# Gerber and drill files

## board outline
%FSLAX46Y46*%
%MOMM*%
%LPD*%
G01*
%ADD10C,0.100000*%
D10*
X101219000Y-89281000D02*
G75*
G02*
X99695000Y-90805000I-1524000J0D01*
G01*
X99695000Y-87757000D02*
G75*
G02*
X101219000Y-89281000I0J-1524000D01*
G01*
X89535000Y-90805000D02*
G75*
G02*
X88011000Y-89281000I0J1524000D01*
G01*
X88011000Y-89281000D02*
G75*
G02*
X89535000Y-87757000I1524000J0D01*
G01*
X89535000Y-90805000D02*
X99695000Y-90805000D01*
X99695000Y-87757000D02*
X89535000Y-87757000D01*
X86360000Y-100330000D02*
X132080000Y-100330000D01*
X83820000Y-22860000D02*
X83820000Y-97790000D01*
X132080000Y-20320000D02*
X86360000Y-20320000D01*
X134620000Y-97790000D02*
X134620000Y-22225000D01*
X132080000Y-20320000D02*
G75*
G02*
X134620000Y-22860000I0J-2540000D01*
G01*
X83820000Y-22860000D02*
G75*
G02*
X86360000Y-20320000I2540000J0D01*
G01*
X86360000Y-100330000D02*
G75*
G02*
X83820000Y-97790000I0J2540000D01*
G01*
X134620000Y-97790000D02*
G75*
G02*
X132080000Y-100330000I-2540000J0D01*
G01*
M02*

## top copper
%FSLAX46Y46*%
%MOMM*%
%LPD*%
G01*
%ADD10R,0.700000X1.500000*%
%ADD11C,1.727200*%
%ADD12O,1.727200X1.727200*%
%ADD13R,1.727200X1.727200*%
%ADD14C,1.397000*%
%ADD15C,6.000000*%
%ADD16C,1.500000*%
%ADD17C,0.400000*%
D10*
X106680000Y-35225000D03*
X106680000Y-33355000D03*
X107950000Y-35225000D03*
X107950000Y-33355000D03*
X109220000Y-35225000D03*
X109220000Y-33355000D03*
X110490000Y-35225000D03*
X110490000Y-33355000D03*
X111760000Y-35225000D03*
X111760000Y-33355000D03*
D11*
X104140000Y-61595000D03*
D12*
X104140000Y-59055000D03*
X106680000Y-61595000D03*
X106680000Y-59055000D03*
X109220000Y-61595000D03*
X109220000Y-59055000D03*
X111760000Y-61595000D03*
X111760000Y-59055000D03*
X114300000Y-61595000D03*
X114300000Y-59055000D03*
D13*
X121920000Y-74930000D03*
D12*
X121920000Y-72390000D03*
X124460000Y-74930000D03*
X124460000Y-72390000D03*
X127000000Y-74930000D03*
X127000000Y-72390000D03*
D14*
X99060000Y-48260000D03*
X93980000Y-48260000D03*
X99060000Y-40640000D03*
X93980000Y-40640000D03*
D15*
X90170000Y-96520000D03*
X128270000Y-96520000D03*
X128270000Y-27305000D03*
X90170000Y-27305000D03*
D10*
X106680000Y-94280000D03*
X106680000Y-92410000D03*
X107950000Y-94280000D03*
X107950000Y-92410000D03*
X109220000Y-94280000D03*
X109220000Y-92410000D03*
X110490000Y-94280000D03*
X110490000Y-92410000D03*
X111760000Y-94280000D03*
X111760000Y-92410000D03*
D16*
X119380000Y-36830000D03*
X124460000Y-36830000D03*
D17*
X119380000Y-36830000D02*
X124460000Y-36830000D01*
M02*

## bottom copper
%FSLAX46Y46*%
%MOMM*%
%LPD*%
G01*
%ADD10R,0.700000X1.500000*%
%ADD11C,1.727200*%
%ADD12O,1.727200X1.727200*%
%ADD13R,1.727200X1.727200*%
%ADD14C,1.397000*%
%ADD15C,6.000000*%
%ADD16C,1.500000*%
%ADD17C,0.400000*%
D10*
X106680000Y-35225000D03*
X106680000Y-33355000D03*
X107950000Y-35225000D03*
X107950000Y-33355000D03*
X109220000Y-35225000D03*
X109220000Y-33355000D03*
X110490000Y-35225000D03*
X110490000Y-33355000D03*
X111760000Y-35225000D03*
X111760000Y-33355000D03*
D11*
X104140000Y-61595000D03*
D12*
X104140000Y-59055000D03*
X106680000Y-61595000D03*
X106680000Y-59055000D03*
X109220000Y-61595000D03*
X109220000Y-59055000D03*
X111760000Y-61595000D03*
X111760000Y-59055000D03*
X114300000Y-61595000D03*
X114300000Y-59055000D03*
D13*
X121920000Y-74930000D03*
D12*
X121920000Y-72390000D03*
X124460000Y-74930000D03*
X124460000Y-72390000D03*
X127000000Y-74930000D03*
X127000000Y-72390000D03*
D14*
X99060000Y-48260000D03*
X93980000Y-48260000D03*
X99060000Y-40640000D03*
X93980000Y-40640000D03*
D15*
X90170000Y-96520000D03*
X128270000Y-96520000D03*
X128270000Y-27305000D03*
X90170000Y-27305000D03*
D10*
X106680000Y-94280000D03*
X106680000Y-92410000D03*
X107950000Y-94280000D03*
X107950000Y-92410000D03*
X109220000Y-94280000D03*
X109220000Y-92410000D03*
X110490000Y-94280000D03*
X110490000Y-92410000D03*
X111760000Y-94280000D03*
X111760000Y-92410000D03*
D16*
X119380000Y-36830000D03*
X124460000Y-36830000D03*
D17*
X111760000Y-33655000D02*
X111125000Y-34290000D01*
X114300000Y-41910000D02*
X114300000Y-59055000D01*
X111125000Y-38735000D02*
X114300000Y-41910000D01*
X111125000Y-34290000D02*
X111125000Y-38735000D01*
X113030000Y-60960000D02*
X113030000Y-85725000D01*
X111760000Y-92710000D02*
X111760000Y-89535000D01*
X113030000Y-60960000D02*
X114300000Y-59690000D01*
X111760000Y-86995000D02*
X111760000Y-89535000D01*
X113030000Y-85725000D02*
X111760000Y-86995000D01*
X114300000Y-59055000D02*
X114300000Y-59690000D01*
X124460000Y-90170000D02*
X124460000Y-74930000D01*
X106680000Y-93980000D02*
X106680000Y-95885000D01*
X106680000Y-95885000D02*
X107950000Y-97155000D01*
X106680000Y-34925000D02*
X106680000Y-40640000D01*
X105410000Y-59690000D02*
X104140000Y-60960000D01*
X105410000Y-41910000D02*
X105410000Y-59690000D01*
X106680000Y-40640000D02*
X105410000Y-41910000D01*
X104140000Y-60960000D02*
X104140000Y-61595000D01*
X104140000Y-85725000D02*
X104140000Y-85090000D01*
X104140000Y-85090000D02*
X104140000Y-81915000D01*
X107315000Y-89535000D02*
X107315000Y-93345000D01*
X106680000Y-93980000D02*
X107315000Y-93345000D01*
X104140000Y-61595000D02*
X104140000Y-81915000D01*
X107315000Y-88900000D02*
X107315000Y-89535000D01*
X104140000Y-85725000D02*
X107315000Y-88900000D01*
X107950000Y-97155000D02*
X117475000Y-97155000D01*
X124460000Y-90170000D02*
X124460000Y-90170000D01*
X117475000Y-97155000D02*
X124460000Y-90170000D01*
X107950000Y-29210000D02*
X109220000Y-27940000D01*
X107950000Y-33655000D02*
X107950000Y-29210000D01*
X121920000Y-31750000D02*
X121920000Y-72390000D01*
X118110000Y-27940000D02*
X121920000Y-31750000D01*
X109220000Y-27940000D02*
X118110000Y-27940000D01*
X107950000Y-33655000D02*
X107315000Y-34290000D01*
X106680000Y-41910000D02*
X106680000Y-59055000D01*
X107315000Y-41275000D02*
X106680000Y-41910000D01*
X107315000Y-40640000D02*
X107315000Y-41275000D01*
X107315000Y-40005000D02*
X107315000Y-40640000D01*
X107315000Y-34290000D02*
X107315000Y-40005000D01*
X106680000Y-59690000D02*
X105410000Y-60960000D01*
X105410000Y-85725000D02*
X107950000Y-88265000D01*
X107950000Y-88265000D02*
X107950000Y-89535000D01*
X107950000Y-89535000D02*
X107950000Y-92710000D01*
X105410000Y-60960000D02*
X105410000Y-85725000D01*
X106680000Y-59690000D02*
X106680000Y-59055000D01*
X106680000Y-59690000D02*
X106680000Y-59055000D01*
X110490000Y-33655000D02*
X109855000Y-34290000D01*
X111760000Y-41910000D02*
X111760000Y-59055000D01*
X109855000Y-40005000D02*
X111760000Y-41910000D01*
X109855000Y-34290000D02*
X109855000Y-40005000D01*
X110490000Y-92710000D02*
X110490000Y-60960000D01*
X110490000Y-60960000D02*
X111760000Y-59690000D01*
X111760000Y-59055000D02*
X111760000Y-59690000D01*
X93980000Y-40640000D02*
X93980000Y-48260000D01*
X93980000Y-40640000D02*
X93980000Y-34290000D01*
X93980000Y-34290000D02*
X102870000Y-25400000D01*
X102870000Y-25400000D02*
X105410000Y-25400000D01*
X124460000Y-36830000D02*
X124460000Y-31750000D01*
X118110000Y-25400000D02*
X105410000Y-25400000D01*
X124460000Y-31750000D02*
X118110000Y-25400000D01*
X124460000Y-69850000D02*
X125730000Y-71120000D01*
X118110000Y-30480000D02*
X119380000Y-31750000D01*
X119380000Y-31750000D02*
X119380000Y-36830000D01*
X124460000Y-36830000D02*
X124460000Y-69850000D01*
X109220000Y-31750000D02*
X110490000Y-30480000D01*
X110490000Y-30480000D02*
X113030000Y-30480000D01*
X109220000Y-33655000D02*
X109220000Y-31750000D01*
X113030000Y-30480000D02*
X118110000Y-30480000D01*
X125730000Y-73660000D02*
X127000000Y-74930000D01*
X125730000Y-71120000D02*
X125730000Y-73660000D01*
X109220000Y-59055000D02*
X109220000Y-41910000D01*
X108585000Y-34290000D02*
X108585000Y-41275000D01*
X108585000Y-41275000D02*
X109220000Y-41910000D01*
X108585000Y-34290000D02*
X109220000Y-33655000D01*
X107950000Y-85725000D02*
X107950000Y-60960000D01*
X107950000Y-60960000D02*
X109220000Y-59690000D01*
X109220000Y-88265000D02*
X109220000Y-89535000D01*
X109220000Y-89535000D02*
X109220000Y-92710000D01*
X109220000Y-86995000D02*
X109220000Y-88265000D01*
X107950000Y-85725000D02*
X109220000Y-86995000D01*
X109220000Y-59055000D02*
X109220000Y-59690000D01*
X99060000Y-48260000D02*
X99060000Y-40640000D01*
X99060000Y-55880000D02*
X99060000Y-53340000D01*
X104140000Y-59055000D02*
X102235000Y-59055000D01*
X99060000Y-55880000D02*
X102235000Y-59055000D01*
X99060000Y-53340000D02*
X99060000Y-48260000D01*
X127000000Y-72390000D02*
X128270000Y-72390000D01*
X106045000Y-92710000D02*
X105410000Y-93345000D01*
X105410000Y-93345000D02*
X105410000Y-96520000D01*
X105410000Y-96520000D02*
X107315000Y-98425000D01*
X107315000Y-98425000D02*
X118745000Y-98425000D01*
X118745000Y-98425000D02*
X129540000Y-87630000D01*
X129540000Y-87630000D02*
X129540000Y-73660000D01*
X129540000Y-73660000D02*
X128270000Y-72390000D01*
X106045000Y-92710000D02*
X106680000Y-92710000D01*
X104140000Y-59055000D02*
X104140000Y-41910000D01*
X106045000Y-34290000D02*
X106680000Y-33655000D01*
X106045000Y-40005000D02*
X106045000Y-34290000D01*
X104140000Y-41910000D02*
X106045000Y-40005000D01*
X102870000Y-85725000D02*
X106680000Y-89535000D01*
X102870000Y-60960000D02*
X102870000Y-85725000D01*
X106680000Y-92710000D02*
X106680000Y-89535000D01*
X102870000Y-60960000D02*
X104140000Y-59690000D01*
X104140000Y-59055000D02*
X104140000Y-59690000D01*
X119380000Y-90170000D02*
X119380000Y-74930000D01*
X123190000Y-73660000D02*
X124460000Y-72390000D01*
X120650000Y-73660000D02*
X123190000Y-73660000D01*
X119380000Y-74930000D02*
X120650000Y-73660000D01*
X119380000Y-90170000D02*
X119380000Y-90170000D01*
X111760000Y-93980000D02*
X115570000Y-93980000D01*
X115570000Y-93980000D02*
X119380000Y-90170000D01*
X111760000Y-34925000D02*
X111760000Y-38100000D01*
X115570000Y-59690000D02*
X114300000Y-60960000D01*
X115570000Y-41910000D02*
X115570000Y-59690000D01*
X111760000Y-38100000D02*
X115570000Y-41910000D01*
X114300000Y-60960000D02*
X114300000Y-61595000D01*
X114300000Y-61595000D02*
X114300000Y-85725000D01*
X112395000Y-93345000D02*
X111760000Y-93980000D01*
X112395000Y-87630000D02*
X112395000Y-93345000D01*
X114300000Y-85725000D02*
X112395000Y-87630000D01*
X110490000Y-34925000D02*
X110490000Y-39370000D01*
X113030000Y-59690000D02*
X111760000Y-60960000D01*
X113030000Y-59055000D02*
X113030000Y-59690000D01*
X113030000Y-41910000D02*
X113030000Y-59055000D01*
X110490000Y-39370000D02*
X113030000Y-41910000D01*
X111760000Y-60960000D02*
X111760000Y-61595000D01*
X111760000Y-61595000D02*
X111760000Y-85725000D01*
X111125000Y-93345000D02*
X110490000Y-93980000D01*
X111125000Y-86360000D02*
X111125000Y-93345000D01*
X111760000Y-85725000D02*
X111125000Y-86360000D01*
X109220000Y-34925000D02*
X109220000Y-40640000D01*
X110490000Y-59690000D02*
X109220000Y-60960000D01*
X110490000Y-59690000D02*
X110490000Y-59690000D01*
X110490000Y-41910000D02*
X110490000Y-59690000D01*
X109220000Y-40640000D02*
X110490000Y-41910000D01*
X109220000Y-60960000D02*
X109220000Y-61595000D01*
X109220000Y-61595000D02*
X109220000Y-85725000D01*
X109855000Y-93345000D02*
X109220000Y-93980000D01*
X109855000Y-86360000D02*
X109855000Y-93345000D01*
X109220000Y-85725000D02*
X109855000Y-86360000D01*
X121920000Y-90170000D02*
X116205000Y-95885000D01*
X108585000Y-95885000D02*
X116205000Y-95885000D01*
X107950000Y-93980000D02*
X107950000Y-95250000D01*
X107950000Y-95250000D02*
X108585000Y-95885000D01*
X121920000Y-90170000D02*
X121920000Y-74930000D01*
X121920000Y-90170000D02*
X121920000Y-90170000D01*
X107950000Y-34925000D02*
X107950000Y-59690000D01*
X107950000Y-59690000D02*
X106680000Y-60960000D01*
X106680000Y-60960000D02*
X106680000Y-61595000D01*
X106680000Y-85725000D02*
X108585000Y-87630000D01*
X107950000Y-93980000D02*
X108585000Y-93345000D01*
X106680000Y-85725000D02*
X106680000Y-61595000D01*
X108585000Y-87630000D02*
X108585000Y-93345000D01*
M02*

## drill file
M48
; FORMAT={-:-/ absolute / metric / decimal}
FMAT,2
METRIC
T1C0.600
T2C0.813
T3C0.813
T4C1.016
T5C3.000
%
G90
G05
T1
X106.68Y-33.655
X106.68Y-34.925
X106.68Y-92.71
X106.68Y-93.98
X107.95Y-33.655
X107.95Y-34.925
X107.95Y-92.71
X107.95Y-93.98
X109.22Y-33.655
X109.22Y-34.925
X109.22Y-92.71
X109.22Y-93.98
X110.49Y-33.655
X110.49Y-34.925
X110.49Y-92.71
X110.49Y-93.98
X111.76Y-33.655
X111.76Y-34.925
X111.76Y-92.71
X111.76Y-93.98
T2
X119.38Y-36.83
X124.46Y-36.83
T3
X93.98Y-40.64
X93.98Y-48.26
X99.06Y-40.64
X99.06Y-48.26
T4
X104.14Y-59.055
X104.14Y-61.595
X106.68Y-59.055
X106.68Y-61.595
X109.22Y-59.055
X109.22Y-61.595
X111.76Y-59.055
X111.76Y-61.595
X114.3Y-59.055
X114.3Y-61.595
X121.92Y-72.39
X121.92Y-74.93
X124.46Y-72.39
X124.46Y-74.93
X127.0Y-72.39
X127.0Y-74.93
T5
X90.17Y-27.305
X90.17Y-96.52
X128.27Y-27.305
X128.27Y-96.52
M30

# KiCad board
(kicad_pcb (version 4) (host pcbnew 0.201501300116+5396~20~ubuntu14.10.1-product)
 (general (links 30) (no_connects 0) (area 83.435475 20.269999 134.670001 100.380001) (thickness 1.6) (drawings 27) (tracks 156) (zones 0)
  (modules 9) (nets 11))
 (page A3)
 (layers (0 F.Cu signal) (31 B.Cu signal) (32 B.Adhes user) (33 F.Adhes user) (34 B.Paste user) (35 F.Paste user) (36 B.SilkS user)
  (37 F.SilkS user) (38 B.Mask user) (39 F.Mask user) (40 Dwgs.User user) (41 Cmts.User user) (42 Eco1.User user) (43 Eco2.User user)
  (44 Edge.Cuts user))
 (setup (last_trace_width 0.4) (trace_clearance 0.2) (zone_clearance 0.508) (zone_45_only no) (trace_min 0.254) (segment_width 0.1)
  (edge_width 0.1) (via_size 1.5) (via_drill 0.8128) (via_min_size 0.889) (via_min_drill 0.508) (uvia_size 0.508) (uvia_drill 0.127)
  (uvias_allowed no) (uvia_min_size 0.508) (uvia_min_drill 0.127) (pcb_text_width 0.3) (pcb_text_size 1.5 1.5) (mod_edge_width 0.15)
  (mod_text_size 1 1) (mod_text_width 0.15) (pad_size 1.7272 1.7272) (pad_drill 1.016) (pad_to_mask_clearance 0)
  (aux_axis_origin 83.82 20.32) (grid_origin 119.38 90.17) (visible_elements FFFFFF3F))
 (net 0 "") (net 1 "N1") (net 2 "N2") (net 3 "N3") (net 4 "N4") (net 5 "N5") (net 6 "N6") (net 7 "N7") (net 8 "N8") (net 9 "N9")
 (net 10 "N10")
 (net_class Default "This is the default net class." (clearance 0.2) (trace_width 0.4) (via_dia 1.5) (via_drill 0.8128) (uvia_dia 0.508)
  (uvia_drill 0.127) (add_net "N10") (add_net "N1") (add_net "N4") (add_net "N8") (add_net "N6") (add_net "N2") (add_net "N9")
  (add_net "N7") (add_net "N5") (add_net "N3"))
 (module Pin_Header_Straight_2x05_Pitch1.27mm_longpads (layer F.Cu) (at 109.22 34.29)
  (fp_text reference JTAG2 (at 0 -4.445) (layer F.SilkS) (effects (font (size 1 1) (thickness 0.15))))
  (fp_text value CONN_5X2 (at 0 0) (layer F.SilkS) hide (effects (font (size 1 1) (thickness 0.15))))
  (pad 1 thru_hole rect (at -2.54 0.635) (size 0.7 1.5) (drill 0.6 (offset 0 0.3)) (layers *.Cu *.Mask F.SilkS) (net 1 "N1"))
  (pad 2 thru_hole rect (at -2.54 -0.635) (size 0.7 1.5) (drill 0.6 (offset 0 -0.3)) (layers *.Cu *.Mask F.SilkS) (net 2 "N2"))
  (pad 3 thru_hole rect (at -1.27 0.635) (size 0.7 1.5) (drill 0.6 (offset 0 0.3)) (layers *.Cu *.Mask F.SilkS) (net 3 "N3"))
  (pad 4 thru_hole rect (at -1.27 -0.635) (size 0.7 1.5) (drill 0.6 (offset 0 -0.3)) (layers *.Cu *.Mask F.SilkS) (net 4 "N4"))
  (pad 5 thru_hole rect (at 0 0.635) (size 0.7 1.5) (drill 0.6 (offset 0 0.3)) (layers *.Cu *.Mask F.SilkS) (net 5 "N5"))
  (pad 6 thru_hole rect (at 0 -0.635) (size 0.7 1.5) (drill 0.6 (offset 0 -0.3)) (layers *.Cu *.Mask F.SilkS) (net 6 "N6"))
  (pad 7 thru_hole rect (at 1.27 0.635) (size 0.7 1.5) (drill 0.6 (offset 0 0.3)) (layers *.Cu *.Mask F.SilkS) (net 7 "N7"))
  (pad 8 thru_hole rect (at 1.27 -0.635) (size 0.7 1.5) (drill 0.6 (offset 0 -0.3)) (layers *.Cu *.Mask F.SilkS) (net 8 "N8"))
  (pad 9 thru_hole rect (at 2.54 0.635) (size 0.7 1.5) (drill 0.6 (offset 0 0.3)) (layers *.Cu *.Mask F.SilkS) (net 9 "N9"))
  (pad 10 thru_hole rect (at 2.54 -0.635) (size 0.7 1.5) (drill 0.6 (offset 0 -0.3)) (layers *.Cu *.Mask F.SilkS) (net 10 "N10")))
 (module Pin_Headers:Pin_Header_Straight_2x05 (layer F.Cu) (at 109.22 60.325)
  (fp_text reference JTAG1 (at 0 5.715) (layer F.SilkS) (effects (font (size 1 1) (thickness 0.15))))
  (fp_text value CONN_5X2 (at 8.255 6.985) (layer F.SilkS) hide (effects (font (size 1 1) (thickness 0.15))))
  (pad 1 thru_hole circle (at -5.08 1.27) (size 1.7272 1.7272) (drill 1.016) (layers *.Cu *.Mask F.SilkS) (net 1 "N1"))
  (pad 2 thru_hole oval (at -5.08 -1.27) (size 1.7272 1.7272) (drill 1.016) (layers *.Cu *.Mask F.SilkS) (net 2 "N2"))
  (pad 3 thru_hole oval (at -2.54 1.27) (size 1.7272 1.7272) (drill 1.016) (layers *.Cu *.Mask F.SilkS) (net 3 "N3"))
  (pad 4 thru_hole oval (at -2.54 -1.27) (size 1.7272 1.7272) (drill 1.016) (layers *.Cu *.Mask F.SilkS) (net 4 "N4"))
  (pad 5 thru_hole oval (at 0 1.27) (size 1.7272 1.7272) (drill 1.016) (layers *.Cu *.Mask F.SilkS) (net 5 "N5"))
  (pad 6 thru_hole oval (at 0 -1.27) (size 1.7272 1.7272) (drill 1.016) (layers *.Cu *.Mask F.SilkS) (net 6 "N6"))
  (pad 7 thru_hole oval (at 2.54 1.27) (size 1.7272 1.7272) (drill 1.016) (layers *.Cu *.Mask F.SilkS) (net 7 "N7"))
  (pad 8 thru_hole oval (at 2.54 -1.27) (size 1.7272 1.7272) (drill 1.016) (layers *.Cu *.Mask F.SilkS) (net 8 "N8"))
  (pad 9 thru_hole oval (at 5.08 1.27) (size 1.7272 1.7272) (drill 1.016) (layers *.Cu *.Mask F.SilkS) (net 9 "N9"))
  (pad 10 thru_hole oval (at 5.08 -1.27) (size 1.7272 1.7272) (drill 1.016) (layers *.Cu *.Mask F.SilkS) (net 10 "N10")))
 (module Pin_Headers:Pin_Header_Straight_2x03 (layer F.Cu) (at 124.46 73.66)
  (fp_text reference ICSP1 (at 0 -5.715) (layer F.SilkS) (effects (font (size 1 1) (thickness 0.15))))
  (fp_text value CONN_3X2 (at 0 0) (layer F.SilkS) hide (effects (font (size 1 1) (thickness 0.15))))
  (pad 1 thru_hole rect (at -2.54 1.27) (size 1.7272 1.7272) (drill 1.016) (layers *.Cu *.Mask F.SilkS) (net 3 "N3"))
  (pad 2 thru_hole oval (at -2.54 -1.27) (size 1.7272 1.7272) (drill 1.016) (layers *.Cu *.Mask F.SilkS) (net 4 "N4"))
  (pad 3 thru_hole oval (at 0 1.27) (size 1.7272 1.7272) (drill 1.016) (layers *.Cu *.Mask F.SilkS) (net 1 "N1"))
  (pad 4 thru_hole oval (at 0 -1.27) (size 1.7272 1.7272) (drill 1.016) (layers *.Cu *.Mask F.SilkS) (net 9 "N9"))
  (pad 5 thru_hole oval (at 2.54 1.27) (size 1.7272 1.7272) (drill 1.016) (layers *.Cu *.Mask F.SilkS) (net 6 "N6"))
  (pad 6 thru_hole oval (at 2.54 -1.27) (size 1.7272 1.7272) (drill 1.016) (layers *.Cu *.Mask F.SilkS) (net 2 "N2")))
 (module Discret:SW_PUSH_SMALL (layer F.Cu) (at 96.52 44.45 270)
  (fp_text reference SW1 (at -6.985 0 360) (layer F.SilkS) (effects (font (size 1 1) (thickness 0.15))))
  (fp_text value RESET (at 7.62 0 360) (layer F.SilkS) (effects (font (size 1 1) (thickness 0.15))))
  (pad 1 thru_hole circle (at 3.81 -2.54 270) (size 1.397 1.397) (drill 0.8128) (layers *.Cu *.Mask F.SilkS) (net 2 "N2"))
  (pad 2 thru_hole circle (at 3.81 2.54 270) (size 1.397 1.397) (drill 0.8128) (layers *.Cu *.Mask F.SilkS) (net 6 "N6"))
  (pad 1 thru_hole circle (at -3.81 -2.54 270) (size 1.397 1.397) (drill 0.8128) (layers *.Cu *.Mask F.SilkS) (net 2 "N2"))
  (pad 2 thru_hole circle (at -3.81 2.54 270) (size 1.397 1.397) (drill 0.8128) (layers *.Cu *.Mask F.SilkS) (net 6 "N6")))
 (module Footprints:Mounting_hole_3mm (layer F.Cu) (at 90.17 96.52)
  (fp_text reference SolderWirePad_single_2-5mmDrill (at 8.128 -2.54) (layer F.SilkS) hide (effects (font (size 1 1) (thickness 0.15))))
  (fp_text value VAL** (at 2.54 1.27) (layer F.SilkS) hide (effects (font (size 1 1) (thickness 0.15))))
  (pad 1 thru_hole circle (at 0 0) (size 6 6) (drill 3) (layers *.Cu *.Mask F.SilkS)))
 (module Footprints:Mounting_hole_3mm (layer F.Cu) (at 128.27 96.52)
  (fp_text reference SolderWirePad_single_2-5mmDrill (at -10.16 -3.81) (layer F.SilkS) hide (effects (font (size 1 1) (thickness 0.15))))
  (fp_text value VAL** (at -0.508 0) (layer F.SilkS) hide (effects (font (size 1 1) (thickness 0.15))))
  (pad 1 thru_hole circle (at 0 0) (size 6 6) (drill 3) (layers *.Cu *.Mask F.SilkS)))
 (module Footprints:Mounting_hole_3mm (layer F.Cu) (at 128.27 27.305)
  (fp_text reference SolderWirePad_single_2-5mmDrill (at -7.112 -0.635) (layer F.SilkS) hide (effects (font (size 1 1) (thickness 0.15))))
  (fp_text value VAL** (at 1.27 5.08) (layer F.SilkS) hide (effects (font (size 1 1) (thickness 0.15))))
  (pad 1 thru_hole circle (at 0 0) (size 6 6) (drill 3) (layers *.Cu *.Mask F.SilkS)))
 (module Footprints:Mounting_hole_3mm (layer F.Cu) (at 90.17 27.305)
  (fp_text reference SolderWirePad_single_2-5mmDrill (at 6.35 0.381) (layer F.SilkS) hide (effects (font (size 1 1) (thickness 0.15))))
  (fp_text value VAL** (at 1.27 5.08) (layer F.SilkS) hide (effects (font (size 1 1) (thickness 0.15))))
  (pad 1 thru_hole circle (at 0 0) (size 6 6) (drill 3) (layers *.Cu *.Mask F.SilkS)))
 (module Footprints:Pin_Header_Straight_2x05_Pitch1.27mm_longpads (layer F.Cu) (at 109.22 93.345)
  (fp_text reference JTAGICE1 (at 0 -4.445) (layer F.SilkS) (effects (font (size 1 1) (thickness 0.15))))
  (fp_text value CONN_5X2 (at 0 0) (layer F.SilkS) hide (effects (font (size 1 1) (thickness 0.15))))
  (pad 1 thru_hole rect (at -2.54 0.635) (size 0.7 1.5) (drill 0.6 (offset 0 0.3)) (layers *.Cu *.Mask F.SilkS) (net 1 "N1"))
  (pad 2 thru_hole rect (at -2.54 -0.635) (size 0.7 1.5) (drill 0.6 (offset 0 -0.3)) (layers *.Cu *.Mask F.SilkS) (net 2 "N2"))
  (pad 3 thru_hole rect (at -1.27 0.635) (size 0.7 1.5) (drill 0.6 (offset 0 0.3)) (layers *.Cu *.Mask F.SilkS) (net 3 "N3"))
  (pad 4 thru_hole rect (at -1.27 -0.635) (size 0.7 1.5) (drill 0.6 (offset 0 -0.3)) (layers *.Cu *.Mask F.SilkS) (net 4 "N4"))
  (pad 5 thru_hole rect (at 0 0.635) (size 0.7 1.5) (drill 0.6 (offset 0 0.3)) (layers *.Cu *.Mask F.SilkS) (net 5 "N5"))
  (pad 6 thru_hole rect (at 0 -0.635) (size 0.7 1.5) (drill 0.6 (offset 0 -0.3)) (layers *.Cu *.Mask F.SilkS) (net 6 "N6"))
  (pad 7 thru_hole rect (at 1.27 0.635) (size 0.7 1.5) (drill 0.6 (offset 0 0.3)) (layers *.Cu *.Mask F.SilkS) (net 7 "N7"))
  (pad 8 thru_hole rect (at 1.27 -0.635) (size 0.7 1.5) (drill 0.6 (offset 0 -0.3)) (layers *.Cu *.Mask F.SilkS) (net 8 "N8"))
  (pad 9 thru_hole rect (at 2.54 0.635) (size 0.7 1.5) (drill 0.6 (offset 0 0.3)) (layers *.Cu *.Mask F.SilkS) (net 9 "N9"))
  (pad 10 thru_hole rect (at 2.54 -0.635) (size 0.7 1.5) (drill 0.6 (offset 0 -0.3)) (layers *.Cu *.Mask F.SilkS) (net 10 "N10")))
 (gr_arc (start 99.695 89.281) (end 101.219 89.281) (angle 90) (layer Edge.Cuts) (width 0.1))
 (gr_arc (start 99.695 89.281) (end 99.695 87.757) (angle 90) (layer Edge.Cuts) (width 0.1))
 (gr_arc (start 89.535 89.281) (end 89.535 90.805) (angle 90) (layer Edge.Cuts) (width 0.1))
 (gr_arc (start 89.535 89.281) (end 88.011 89.281) (angle 90) (layer Edge.Cuts) (width 0.1))
 (gr_line (start 89.535 90.805) (end 99.695 90.805) (angle 90) (layer Edge.Cuts) (width 0.1))
 (gr_line (start 99.695 87.757) (end 89.535 87.757) (angle 90) (layer Edge.Cuts) (width 0.1))
 (gr_line (start 86.36 100.33) (end 132.08 100.33) (angle 90) (layer Edge.Cuts) (width 0.1))
 (gr_line (start 83.82 22.86) (end 83.82 97.79) (angle 90) (layer Edge.Cuts) (width 0.1))
 (gr_line (start 132.08 20.32) (end 86.36 20.32) (angle 90) (layer Edge.Cuts) (width 0.1))
 (gr_line (start 134.62 97.79) (end 134.62 22.225) (angle 90) (layer Edge.Cuts) (width 0.1))
 (gr_arc (start 132.08 22.86) (end 132.08 20.32) (angle 90) (layer Edge.Cuts) (width 0.1))
 (gr_arc (start 86.36 22.86) (end 83.82 22.86) (angle 90) (layer Edge.Cuts) (width 0.1))
 (gr_arc (start 86.36 97.79) (end 86.36 100.33) (angle 90) (layer Edge.Cuts) (width 0.1))
 (gr_arc (start 132.08 97.79) (end 134.62 97.79) (angle 90) (layer Edge.Cuts) (width 0.1))
 (segment (start 111.76 33.655) (end 111.125 34.29) (width 0.4) (layer B.Cu) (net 10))
 (segment (start 114.3 41.91) (end 114.3 59.055) (width 0.4) (layer B.Cu) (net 10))
 (segment (start 111.125 38.735) (end 114.3 41.91) (width 0.4) (layer B.Cu) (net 10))
 (segment (start 111.125 34.29) (end 111.125 38.735) (width 0.4) (layer B.Cu) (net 10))
 (segment (start 113.03 60.96) (end 113.03 85.725) (width 0.4) (layer B.Cu) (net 10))
 (segment (start 111.76 92.71) (end 111.76 89.535) (width 0.4) (layer B.Cu) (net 10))
 (segment (start 113.03 60.96) (end 114.3 59.69) (width 0.4) (layer B.Cu) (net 10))
 (segment (start 111.76 86.995) (end 111.76 89.535) (width 0.4) (layer B.Cu) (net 10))
 (segment (start 113.03 85.725) (end 111.76 86.995) (width 0.4) (layer B.Cu) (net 10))
 (segment (start 114.3 59.055) (end 114.3 59.69) (width 0.4) (layer B.Cu) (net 10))
 (segment (start 124.46 90.17) (end 124.46 74.93) (width 0.4) (layer B.Cu) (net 1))
 (segment (start 106.68 93.98) (end 106.68 95.885) (width 0.4) (layer B.Cu) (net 1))
 (segment (start 106.68 95.885) (end 107.95 97.155) (width 0.4) (layer B.Cu) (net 1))
 (segment (start 106.68 34.925) (end 106.68 40.64) (width 0.4) (layer B.Cu) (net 1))
 (segment (start 105.41 59.69) (end 104.14 60.96) (width 0.4) (layer B.Cu) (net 1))
 (segment (start 105.41 41.91) (end 105.41 59.69) (width 0.4) (layer B.Cu) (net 1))
 (segment (start 106.68 40.64) (end 105.41 41.91) (width 0.4) (layer B.Cu) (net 1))
 (segment (start 104.14 60.96) (end 104.14 61.595) (width 0.4) (layer B.Cu) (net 1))
 (segment (start 104.14 85.725) (end 104.14 85.09) (width 0.4) (layer B.Cu) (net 1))
 (segment (start 104.14 85.09) (end 104.14 81.915) (width 0.4) (layer B.Cu) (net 1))
 (segment (start 107.315 89.535) (end 107.315 93.345) (width 0.4) (layer B.Cu) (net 1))
 (segment (start 106.68 93.98) (end 107.315 93.345) (width 0.4) (layer B.Cu) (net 1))
 (segment (start 104.14 61.595) (end 104.14 81.915) (width 0.4) (layer B.Cu) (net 1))
 (segment (start 107.315 88.9) (end 107.315 89.535) (width 0.4) (layer B.Cu) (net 1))
 (segment (start 104.14 85.725) (end 107.315 88.9) (width 0.4) (layer B.Cu) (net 1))
 (segment (start 107.95 97.155) (end 117.475 97.155) (width 0.4) (layer B.Cu) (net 1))
 (segment (start 124.46 90.17) (end 124.46 90.17) (width 0.4) (layer B.Cu) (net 1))
 (segment (start 117.475 97.155) (end 124.46 90.17) (width 0.4) (layer B.Cu) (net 1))
 (segment (start 107.95 29.21) (end 109.22 27.94) (width 0.4) (layer B.Cu) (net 4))
 (segment (start 107.95 33.655) (end 107.95 29.21) (width 0.4) (layer B.Cu) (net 4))
 (segment (start 121.92 31.75) (end 121.92 72.39) (width 0.4) (layer B.Cu) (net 4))
 (segment (start 118.11 27.94) (end 121.92 31.75) (width 0.4) (layer B.Cu) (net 4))
 (segment (start 109.22 27.94) (end 118.11 27.94) (width 0.4) (layer B.Cu) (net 4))
 (segment (start 107.95 33.655) (end 107.315 34.29) (width 0.4) (layer B.Cu) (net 4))
 (segment (start 106.68 41.91) (end 106.68 59.055) (width 0.4) (layer B.Cu) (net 4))
 (segment (start 107.315 41.275) (end 106.68 41.91) (width 0.4) (layer B.Cu) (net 4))
 (segment (start 107.315 40.64) (end 107.315 41.275) (width 0.4) (layer B.Cu) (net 4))
 (segment (start 107.315 40.005) (end 107.315 40.64) (width 0.4) (layer B.Cu) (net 4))
 (segment (start 107.315 34.29) (end 107.315 40.005) (width 0.4) (layer B.Cu) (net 4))
 (segment (start 106.68 59.69) (end 105.41 60.96) (width 0.4) (layer B.Cu) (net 4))
 (segment (start 105.41 85.725) (end 107.95 88.265) (width 0.4) (layer B.Cu) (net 4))
 (segment (start 107.95 88.265) (end 107.95 89.535) (width 0.4) (layer B.Cu) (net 4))
 (segment (start 107.95 89.535) (end 107.95 92.71) (width 0.4) (layer B.Cu) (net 4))
 (segment (start 105.41 60.96) (end 105.41 85.725) (width 0.4) (layer B.Cu) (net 4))
 (segment (start 106.68 59.69) (end 106.68 59.055) (width 0.4) (layer B.Cu) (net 4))
 (segment (start 106.68 59.69) (end 106.68 59.055) (width 0.4) (layer B.Cu) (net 4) (status 30))
 (segment (start 110.49 33.655) (end 109.855 34.29) (width 0.4) (layer B.Cu) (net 8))
 (segment (start 111.76 41.91) (end 111.76 59.055) (width 0.4) (layer B.Cu) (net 8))
 (segment (start 109.855 40.005) (end 111.76 41.91) (width 0.4) (layer B.Cu) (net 8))
 (segment (start 109.855 34.29) (end 109.855 40.005) (width 0.4) (layer B.Cu) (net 8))
 (segment (start 110.49 92.71) (end 110.49 60.96) (width 0.4) (layer B.Cu) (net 8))
 (segment (start 110.49 60.96) (end 111.76 59.69) (width 0.4) (layer B.Cu) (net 8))
 (segment (start 111.76 59.055) (end 111.76 59.69) (width 0.4) (layer B.Cu) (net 8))
 (segment (start 93.98 40.64) (end 93.98 48.26) (width 0.4) (layer B.Cu) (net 6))
 (segment (start 93.98 40.64) (end 93.98 34.29) (width 0.4) (layer B.Cu) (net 6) (status 10))
 (segment (start 93.98 34.29) (end 102.87 25.4) (width 0.4) (layer B.Cu) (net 6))
 (segment (start 102.87 25.4) (end 105.41 25.4) (width 0.4) (layer B.Cu) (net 6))
 (segment (start 124.46 36.83) (end 124.46 31.75) (width 0.4) (layer B.Cu) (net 6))
 (segment (start 118.11 25.4) (end 105.41 25.4) (width 0.4) (layer B.Cu) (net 6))
 (segment (start 124.46 31.75) (end 118.11 25.4) (width 0.4) (layer B.Cu) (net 6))
 (segment (start 124.46 69.85) (end 125.73 71.12) (width 0.4) (layer B.Cu) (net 6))
 (segment (start 118.11 30.48) (end 119.38 31.75) (width 0.4) (layer B.Cu) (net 6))
 (segment (start 119.38 31.75) (end 119.38 36.83) (width 0.4) (layer B.Cu) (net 6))
 (via (at 119.38 36.83) (size 1.5) (layers F.Cu B.Cu) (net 6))
 (segment (start 119.38 36.83) (end 124.46 36.83) (width 0.4) (layer F.Cu) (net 6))
 (via (at 124.46 36.83) (size 1.5) (layers F.Cu B.Cu) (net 6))
 (segment (start 124.46 36.83) (end 124.46 69.85) (width 0.4) (layer B.Cu) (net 6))
 (segment (start 109.22 31.75) (end 110.49 30.48) (width 0.4) (layer B.Cu) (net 6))
 (segment (start 110.49 30.48) (end 113.03 30.48) (width 0.4) (layer B.Cu) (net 6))
 (segment (start 109.22 33.655) (end 109.22 31.75) (width 0.4) (layer B.Cu) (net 6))
 (segment (start 113.03 30.48) (end 118.11 30.48) (width 0.4) (layer B.Cu) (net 6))
 (segment (start 125.73 73.66) (end 127 74.93) (width 0.4) (layer B.Cu) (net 6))
 (segment (start 125.73 71.12) (end 125.73 73.66) (width 0.4) (layer B.Cu) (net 6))
 (segment (start 109.22 59.055) (end 109.22 41.91) (width 0.4) (layer B.Cu) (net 6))
 (segment (start 108.585 34.29) (end 108.585 41.275) (width 0.4) (layer B.Cu) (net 6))
 (segment (start 108.585 41.275) (end 109.22 41.91) (width 0.4) (layer B.Cu) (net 6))
 (segment (start 108.585 34.29) (end 109.22 33.655) (width 0.4) (layer B.Cu) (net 6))
 (segment (start 107.95 85.725) (end 107.95 60.96) (width 0.4) (layer B.Cu) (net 6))
 (segment (start 107.95 60.96) (end 109.22 59.69) (width 0.4) (layer B.Cu) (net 6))
 (segment (start 109.22 88.265) (end 109.22 89.535) (width 0.4) (layer B.Cu) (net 6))
 (segment (start 109.22 89.535) (end 109.22 92.71) (width 0.4) (layer B.Cu) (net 6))
 (segment (start 109.22 86.995) (end 109.22 88.265) (width 0.4) (layer B.Cu) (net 6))
 (segment (start 107.95 85.725) (end 109.22 86.995) (width 0.4) (layer B.Cu) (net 6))
 (segment (start 109.22 59.055) (end 109.22 59.69) (width 0.4) (layer B.Cu) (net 6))
 (segment (start 99.06 48.26) (end 99.06 40.64) (width 0.4) (layer B.Cu) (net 2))
 (segment (start 99.06 55.88) (end 99.06 53.34) (width 0.4) (layer B.Cu) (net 2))
 (segment (start 104.14 59.055) (end 102.235 59.055) (width 0.4) (layer B.Cu) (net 2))
 (segment (start 99.06 55.88) (end 102.235 59.055) (width 0.4) (layer B.Cu) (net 2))
 (segment (start 99.06 53.34) (end 99.06 48.26) (width 0.4) (layer B.Cu) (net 2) (status 10))
 (segment (start 127 72.39) (end 128.27 72.39) (width 0.4) (layer B.Cu) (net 2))
 (segment (start 106.045 92.71) (end 105.41 93.345) (width 0.4) (layer B.Cu) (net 2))
 (segment (start 105.41 93.345) (end 105.41 96.52) (width 0.4) (layer B.Cu) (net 2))
 (segment (start 105.41 96.52) (end 107.315 98.425) (width 0.4) (layer B.Cu) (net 2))
 (segment (start 107.315 98.425) (end 118.745 98.425) (width 0.4) (layer B.Cu) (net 2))
 (segment (start 118.745 98.425) (end 129.54 87.63) (width 0.4) (layer B.Cu) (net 2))
 (segment (start 129.54 87.63) (end 129.54 73.66) (width 0.4) (layer B.Cu) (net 2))
 (segment (start 129.54 73.66) (end 128.27 72.39) (width 0.4) (layer B.Cu) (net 2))
 (segment (start 106.045 92.71) (end 106.68 92.71) (width 0.4) (layer B.Cu) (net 2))
 (segment (start 104.14 59.055) (end 104.14 41.91) (width 0.4) (layer B.Cu) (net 2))
 (segment (start 106.045 34.29) (end 106.68 33.655) (width 0.4) (layer B.Cu) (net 2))
 (segment (start 106.045 40.005) (end 106.045 34.29) (width 0.4) (layer B.Cu) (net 2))
 (segment (start 104.14 41.91) (end 106.045 40.005) (width 0.4) (layer B.Cu) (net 2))
 (segment (start 102.87 85.725) (end 106.68 89.535) (width 0.4) (layer B.Cu) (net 2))
 (segment (start 102.87 60.96) (end 102.87 85.725) (width 0.4) (layer B.Cu) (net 2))
 (segment (start 106.68 92.71) (end 106.68 89.535) (width 0.4) (layer B.Cu) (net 2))
 (segment (start 102.87 60.96) (end 104.14 59.69) (width 0.4) (layer B.Cu) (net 2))
 (segment (start 104.14 59.055) (end 104.14 59.69) (width 0.4) (layer B.Cu) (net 2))
 (segment (start 119.38 90.17) (end 119.38 74.93) (width 0.4) (layer B.Cu) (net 9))
 (segment (start 123.19 73.66) (end 124.46 72.39) (width 0.4) (layer B.Cu) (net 9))
 (segment (start 120.65 73.66) (end 123.19 73.66) (width 0.4) (layer B.Cu) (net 9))
 (segment (start 119.38 74.93) (end 120.65 73.66) (width 0.4) (layer B.Cu) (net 9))
 (segment (start 119.38 90.17) (end 119.38 90.17) (width 0.4) (layer B.Cu) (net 9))
 (segment (start 111.76 93.98) (end 115.57 93.98) (width 0.4) (layer B.Cu) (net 9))
 (segment (start 115.57 93.98) (end 119.38 90.17) (width 0.4) (layer B.Cu) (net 9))
 (segment (start 111.76 34.925) (end 111.76 38.1) (width 0.4) (layer B.Cu) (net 9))
 (segment (start 115.57 59.69) (end 114.3 60.96) (width 0.4) (layer B.Cu) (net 9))
 (segment (start 115.57 41.91) (end 115.57 59.69) (width 0.4) (layer B.Cu) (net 9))
 (segment (start 111.76 38.1) (end 115.57 41.91) (width 0.4) (layer B.Cu) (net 9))
 (segment (start 114.3 60.96) (end 114.3 61.595) (width 0.4) (layer B.Cu) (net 9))
 (segment (start 114.3 61.595) (end 114.3 85.725) (width 0.4) (layer B.Cu) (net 9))
 (segment (start 112.395 93.345) (end 111.76 93.98) (width 0.4) (layer B.Cu) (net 9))
 (segment (start 112.395 87.63) (end 112.395 93.345) (width 0.4) (layer B.Cu) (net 9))
 (segment (start 114.3 85.725) (end 112.395 87.63) (width 0.4) (layer B.Cu) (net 9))
 (segment (start 110.49 34.925) (end 110.49 39.37) (width 0.4) (layer B.Cu) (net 7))
 (segment (start 113.03 59.69) (end 111.76 60.96) (width 0.4) (layer B.Cu) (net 7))
 (segment (start 113.03 59.055) (end 113.03 59.69) (width 0.4) (layer B.Cu) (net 7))
 (segment (start 113.03 41.91) (end 113.03 59.055) (width 0.4) (layer B.Cu) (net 7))
 (segment (start 110.49 39.37) (end 113.03 41.91) (width 0.4) (layer B.Cu) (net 7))
 (segment (start 111.76 60.96) (end 111.76 61.595) (width 0.4) (layer B.Cu) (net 7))
 (segment (start 111.76 61.595) (end 111.76 85.725) (width 0.4) (layer B.Cu) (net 7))
 (segment (start 111.125 93.345) (end 110.49 93.98) (width 0.4) (layer B.Cu) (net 7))
 (segment (start 111.125 86.36) (end 111.125 93.345) (width 0.4) (layer B.Cu) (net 7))
 (segment (start 111.76 85.725) (end 111.125 86.36) (width 0.4) (layer B.Cu) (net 7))
 (segment (start 109.22 34.925) (end 109.22 40.64) (width 0.4) (layer B.Cu) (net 5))
 (segment (start 110.49 59.69) (end 109.22 60.96) (width 0.4) (layer B.Cu) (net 5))
 (segment (start 110.49 59.69) (end 110.49 59.69) (width 0.4) (layer B.Cu) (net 5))
 (segment (start 110.49 41.91) (end 110.49 59.69) (width 0.4) (layer B.Cu) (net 5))
 (segment (start 109.22 40.64) (end 110.49 41.91) (width 0.4) (layer B.Cu) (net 5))
 (segment (start 109.22 60.96) (end 109.22 61.595) (width 0.4) (layer B.Cu) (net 5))
 (segment (start 109.22 61.595) (end 109.22 85.725) (width 0.4) (layer B.Cu) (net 5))
 (segment (start 109.855 93.345) (end 109.22 93.98) (width 0.4) (layer B.Cu) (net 5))
 (segment (start 109.855 86.36) (end 109.855 93.345) (width 0.4) (layer B.Cu) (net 5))
 (segment (start 109.22 85.725) (end 109.855 86.36) (width 0.4) (layer B.Cu) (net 5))
 (segment (start 121.92 90.17) (end 116.205 95.885) (width 0.4) (layer B.Cu) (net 3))
 (segment (start 108.585 95.885) (end 116.205 95.885) (width 0.4) (layer B.Cu) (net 3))
 (segment (start 107.95 93.98) (end 107.95 95.25) (width 0.4) (layer B.Cu) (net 3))
 (segment (start 107.95 95.25) (end 108.585 95.885) (width 0.4) (layer B.Cu) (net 3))
 (segment (start 121.92 90.17) (end 121.92 74.93) (width 0.4) (layer B.Cu) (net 3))
 (segment (start 121.92 90.17) (end 121.92 90.17) (width 0.4) (layer B.Cu) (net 3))
 (segment (start 107.95 34.925) (end 107.95 59.69) (width 0.4) (layer B.Cu) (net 3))
 (segment (start 107.95 59.69) (end 106.68 60.96) (width 0.4) (layer B.Cu) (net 3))
 (segment (start 106.68 60.96) (end 106.68 61.595) (width 0.4) (layer B.Cu) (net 3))
 (segment (start 106.68 85.725) (end 108.585 87.63) (width 0.4) (layer B.Cu) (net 3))
 (segment (start 107.95 93.98) (end 108.585 93.345) (width 0.4) (layer B.Cu) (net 3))
 (segment (start 106.68 85.725) (end 106.68 61.595) (width 0.4) (layer B.Cu) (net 3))
 (segment (start 108.585 87.63) (end 108.585 93.345) (width 0.4) (layer B.Cu) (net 3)))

